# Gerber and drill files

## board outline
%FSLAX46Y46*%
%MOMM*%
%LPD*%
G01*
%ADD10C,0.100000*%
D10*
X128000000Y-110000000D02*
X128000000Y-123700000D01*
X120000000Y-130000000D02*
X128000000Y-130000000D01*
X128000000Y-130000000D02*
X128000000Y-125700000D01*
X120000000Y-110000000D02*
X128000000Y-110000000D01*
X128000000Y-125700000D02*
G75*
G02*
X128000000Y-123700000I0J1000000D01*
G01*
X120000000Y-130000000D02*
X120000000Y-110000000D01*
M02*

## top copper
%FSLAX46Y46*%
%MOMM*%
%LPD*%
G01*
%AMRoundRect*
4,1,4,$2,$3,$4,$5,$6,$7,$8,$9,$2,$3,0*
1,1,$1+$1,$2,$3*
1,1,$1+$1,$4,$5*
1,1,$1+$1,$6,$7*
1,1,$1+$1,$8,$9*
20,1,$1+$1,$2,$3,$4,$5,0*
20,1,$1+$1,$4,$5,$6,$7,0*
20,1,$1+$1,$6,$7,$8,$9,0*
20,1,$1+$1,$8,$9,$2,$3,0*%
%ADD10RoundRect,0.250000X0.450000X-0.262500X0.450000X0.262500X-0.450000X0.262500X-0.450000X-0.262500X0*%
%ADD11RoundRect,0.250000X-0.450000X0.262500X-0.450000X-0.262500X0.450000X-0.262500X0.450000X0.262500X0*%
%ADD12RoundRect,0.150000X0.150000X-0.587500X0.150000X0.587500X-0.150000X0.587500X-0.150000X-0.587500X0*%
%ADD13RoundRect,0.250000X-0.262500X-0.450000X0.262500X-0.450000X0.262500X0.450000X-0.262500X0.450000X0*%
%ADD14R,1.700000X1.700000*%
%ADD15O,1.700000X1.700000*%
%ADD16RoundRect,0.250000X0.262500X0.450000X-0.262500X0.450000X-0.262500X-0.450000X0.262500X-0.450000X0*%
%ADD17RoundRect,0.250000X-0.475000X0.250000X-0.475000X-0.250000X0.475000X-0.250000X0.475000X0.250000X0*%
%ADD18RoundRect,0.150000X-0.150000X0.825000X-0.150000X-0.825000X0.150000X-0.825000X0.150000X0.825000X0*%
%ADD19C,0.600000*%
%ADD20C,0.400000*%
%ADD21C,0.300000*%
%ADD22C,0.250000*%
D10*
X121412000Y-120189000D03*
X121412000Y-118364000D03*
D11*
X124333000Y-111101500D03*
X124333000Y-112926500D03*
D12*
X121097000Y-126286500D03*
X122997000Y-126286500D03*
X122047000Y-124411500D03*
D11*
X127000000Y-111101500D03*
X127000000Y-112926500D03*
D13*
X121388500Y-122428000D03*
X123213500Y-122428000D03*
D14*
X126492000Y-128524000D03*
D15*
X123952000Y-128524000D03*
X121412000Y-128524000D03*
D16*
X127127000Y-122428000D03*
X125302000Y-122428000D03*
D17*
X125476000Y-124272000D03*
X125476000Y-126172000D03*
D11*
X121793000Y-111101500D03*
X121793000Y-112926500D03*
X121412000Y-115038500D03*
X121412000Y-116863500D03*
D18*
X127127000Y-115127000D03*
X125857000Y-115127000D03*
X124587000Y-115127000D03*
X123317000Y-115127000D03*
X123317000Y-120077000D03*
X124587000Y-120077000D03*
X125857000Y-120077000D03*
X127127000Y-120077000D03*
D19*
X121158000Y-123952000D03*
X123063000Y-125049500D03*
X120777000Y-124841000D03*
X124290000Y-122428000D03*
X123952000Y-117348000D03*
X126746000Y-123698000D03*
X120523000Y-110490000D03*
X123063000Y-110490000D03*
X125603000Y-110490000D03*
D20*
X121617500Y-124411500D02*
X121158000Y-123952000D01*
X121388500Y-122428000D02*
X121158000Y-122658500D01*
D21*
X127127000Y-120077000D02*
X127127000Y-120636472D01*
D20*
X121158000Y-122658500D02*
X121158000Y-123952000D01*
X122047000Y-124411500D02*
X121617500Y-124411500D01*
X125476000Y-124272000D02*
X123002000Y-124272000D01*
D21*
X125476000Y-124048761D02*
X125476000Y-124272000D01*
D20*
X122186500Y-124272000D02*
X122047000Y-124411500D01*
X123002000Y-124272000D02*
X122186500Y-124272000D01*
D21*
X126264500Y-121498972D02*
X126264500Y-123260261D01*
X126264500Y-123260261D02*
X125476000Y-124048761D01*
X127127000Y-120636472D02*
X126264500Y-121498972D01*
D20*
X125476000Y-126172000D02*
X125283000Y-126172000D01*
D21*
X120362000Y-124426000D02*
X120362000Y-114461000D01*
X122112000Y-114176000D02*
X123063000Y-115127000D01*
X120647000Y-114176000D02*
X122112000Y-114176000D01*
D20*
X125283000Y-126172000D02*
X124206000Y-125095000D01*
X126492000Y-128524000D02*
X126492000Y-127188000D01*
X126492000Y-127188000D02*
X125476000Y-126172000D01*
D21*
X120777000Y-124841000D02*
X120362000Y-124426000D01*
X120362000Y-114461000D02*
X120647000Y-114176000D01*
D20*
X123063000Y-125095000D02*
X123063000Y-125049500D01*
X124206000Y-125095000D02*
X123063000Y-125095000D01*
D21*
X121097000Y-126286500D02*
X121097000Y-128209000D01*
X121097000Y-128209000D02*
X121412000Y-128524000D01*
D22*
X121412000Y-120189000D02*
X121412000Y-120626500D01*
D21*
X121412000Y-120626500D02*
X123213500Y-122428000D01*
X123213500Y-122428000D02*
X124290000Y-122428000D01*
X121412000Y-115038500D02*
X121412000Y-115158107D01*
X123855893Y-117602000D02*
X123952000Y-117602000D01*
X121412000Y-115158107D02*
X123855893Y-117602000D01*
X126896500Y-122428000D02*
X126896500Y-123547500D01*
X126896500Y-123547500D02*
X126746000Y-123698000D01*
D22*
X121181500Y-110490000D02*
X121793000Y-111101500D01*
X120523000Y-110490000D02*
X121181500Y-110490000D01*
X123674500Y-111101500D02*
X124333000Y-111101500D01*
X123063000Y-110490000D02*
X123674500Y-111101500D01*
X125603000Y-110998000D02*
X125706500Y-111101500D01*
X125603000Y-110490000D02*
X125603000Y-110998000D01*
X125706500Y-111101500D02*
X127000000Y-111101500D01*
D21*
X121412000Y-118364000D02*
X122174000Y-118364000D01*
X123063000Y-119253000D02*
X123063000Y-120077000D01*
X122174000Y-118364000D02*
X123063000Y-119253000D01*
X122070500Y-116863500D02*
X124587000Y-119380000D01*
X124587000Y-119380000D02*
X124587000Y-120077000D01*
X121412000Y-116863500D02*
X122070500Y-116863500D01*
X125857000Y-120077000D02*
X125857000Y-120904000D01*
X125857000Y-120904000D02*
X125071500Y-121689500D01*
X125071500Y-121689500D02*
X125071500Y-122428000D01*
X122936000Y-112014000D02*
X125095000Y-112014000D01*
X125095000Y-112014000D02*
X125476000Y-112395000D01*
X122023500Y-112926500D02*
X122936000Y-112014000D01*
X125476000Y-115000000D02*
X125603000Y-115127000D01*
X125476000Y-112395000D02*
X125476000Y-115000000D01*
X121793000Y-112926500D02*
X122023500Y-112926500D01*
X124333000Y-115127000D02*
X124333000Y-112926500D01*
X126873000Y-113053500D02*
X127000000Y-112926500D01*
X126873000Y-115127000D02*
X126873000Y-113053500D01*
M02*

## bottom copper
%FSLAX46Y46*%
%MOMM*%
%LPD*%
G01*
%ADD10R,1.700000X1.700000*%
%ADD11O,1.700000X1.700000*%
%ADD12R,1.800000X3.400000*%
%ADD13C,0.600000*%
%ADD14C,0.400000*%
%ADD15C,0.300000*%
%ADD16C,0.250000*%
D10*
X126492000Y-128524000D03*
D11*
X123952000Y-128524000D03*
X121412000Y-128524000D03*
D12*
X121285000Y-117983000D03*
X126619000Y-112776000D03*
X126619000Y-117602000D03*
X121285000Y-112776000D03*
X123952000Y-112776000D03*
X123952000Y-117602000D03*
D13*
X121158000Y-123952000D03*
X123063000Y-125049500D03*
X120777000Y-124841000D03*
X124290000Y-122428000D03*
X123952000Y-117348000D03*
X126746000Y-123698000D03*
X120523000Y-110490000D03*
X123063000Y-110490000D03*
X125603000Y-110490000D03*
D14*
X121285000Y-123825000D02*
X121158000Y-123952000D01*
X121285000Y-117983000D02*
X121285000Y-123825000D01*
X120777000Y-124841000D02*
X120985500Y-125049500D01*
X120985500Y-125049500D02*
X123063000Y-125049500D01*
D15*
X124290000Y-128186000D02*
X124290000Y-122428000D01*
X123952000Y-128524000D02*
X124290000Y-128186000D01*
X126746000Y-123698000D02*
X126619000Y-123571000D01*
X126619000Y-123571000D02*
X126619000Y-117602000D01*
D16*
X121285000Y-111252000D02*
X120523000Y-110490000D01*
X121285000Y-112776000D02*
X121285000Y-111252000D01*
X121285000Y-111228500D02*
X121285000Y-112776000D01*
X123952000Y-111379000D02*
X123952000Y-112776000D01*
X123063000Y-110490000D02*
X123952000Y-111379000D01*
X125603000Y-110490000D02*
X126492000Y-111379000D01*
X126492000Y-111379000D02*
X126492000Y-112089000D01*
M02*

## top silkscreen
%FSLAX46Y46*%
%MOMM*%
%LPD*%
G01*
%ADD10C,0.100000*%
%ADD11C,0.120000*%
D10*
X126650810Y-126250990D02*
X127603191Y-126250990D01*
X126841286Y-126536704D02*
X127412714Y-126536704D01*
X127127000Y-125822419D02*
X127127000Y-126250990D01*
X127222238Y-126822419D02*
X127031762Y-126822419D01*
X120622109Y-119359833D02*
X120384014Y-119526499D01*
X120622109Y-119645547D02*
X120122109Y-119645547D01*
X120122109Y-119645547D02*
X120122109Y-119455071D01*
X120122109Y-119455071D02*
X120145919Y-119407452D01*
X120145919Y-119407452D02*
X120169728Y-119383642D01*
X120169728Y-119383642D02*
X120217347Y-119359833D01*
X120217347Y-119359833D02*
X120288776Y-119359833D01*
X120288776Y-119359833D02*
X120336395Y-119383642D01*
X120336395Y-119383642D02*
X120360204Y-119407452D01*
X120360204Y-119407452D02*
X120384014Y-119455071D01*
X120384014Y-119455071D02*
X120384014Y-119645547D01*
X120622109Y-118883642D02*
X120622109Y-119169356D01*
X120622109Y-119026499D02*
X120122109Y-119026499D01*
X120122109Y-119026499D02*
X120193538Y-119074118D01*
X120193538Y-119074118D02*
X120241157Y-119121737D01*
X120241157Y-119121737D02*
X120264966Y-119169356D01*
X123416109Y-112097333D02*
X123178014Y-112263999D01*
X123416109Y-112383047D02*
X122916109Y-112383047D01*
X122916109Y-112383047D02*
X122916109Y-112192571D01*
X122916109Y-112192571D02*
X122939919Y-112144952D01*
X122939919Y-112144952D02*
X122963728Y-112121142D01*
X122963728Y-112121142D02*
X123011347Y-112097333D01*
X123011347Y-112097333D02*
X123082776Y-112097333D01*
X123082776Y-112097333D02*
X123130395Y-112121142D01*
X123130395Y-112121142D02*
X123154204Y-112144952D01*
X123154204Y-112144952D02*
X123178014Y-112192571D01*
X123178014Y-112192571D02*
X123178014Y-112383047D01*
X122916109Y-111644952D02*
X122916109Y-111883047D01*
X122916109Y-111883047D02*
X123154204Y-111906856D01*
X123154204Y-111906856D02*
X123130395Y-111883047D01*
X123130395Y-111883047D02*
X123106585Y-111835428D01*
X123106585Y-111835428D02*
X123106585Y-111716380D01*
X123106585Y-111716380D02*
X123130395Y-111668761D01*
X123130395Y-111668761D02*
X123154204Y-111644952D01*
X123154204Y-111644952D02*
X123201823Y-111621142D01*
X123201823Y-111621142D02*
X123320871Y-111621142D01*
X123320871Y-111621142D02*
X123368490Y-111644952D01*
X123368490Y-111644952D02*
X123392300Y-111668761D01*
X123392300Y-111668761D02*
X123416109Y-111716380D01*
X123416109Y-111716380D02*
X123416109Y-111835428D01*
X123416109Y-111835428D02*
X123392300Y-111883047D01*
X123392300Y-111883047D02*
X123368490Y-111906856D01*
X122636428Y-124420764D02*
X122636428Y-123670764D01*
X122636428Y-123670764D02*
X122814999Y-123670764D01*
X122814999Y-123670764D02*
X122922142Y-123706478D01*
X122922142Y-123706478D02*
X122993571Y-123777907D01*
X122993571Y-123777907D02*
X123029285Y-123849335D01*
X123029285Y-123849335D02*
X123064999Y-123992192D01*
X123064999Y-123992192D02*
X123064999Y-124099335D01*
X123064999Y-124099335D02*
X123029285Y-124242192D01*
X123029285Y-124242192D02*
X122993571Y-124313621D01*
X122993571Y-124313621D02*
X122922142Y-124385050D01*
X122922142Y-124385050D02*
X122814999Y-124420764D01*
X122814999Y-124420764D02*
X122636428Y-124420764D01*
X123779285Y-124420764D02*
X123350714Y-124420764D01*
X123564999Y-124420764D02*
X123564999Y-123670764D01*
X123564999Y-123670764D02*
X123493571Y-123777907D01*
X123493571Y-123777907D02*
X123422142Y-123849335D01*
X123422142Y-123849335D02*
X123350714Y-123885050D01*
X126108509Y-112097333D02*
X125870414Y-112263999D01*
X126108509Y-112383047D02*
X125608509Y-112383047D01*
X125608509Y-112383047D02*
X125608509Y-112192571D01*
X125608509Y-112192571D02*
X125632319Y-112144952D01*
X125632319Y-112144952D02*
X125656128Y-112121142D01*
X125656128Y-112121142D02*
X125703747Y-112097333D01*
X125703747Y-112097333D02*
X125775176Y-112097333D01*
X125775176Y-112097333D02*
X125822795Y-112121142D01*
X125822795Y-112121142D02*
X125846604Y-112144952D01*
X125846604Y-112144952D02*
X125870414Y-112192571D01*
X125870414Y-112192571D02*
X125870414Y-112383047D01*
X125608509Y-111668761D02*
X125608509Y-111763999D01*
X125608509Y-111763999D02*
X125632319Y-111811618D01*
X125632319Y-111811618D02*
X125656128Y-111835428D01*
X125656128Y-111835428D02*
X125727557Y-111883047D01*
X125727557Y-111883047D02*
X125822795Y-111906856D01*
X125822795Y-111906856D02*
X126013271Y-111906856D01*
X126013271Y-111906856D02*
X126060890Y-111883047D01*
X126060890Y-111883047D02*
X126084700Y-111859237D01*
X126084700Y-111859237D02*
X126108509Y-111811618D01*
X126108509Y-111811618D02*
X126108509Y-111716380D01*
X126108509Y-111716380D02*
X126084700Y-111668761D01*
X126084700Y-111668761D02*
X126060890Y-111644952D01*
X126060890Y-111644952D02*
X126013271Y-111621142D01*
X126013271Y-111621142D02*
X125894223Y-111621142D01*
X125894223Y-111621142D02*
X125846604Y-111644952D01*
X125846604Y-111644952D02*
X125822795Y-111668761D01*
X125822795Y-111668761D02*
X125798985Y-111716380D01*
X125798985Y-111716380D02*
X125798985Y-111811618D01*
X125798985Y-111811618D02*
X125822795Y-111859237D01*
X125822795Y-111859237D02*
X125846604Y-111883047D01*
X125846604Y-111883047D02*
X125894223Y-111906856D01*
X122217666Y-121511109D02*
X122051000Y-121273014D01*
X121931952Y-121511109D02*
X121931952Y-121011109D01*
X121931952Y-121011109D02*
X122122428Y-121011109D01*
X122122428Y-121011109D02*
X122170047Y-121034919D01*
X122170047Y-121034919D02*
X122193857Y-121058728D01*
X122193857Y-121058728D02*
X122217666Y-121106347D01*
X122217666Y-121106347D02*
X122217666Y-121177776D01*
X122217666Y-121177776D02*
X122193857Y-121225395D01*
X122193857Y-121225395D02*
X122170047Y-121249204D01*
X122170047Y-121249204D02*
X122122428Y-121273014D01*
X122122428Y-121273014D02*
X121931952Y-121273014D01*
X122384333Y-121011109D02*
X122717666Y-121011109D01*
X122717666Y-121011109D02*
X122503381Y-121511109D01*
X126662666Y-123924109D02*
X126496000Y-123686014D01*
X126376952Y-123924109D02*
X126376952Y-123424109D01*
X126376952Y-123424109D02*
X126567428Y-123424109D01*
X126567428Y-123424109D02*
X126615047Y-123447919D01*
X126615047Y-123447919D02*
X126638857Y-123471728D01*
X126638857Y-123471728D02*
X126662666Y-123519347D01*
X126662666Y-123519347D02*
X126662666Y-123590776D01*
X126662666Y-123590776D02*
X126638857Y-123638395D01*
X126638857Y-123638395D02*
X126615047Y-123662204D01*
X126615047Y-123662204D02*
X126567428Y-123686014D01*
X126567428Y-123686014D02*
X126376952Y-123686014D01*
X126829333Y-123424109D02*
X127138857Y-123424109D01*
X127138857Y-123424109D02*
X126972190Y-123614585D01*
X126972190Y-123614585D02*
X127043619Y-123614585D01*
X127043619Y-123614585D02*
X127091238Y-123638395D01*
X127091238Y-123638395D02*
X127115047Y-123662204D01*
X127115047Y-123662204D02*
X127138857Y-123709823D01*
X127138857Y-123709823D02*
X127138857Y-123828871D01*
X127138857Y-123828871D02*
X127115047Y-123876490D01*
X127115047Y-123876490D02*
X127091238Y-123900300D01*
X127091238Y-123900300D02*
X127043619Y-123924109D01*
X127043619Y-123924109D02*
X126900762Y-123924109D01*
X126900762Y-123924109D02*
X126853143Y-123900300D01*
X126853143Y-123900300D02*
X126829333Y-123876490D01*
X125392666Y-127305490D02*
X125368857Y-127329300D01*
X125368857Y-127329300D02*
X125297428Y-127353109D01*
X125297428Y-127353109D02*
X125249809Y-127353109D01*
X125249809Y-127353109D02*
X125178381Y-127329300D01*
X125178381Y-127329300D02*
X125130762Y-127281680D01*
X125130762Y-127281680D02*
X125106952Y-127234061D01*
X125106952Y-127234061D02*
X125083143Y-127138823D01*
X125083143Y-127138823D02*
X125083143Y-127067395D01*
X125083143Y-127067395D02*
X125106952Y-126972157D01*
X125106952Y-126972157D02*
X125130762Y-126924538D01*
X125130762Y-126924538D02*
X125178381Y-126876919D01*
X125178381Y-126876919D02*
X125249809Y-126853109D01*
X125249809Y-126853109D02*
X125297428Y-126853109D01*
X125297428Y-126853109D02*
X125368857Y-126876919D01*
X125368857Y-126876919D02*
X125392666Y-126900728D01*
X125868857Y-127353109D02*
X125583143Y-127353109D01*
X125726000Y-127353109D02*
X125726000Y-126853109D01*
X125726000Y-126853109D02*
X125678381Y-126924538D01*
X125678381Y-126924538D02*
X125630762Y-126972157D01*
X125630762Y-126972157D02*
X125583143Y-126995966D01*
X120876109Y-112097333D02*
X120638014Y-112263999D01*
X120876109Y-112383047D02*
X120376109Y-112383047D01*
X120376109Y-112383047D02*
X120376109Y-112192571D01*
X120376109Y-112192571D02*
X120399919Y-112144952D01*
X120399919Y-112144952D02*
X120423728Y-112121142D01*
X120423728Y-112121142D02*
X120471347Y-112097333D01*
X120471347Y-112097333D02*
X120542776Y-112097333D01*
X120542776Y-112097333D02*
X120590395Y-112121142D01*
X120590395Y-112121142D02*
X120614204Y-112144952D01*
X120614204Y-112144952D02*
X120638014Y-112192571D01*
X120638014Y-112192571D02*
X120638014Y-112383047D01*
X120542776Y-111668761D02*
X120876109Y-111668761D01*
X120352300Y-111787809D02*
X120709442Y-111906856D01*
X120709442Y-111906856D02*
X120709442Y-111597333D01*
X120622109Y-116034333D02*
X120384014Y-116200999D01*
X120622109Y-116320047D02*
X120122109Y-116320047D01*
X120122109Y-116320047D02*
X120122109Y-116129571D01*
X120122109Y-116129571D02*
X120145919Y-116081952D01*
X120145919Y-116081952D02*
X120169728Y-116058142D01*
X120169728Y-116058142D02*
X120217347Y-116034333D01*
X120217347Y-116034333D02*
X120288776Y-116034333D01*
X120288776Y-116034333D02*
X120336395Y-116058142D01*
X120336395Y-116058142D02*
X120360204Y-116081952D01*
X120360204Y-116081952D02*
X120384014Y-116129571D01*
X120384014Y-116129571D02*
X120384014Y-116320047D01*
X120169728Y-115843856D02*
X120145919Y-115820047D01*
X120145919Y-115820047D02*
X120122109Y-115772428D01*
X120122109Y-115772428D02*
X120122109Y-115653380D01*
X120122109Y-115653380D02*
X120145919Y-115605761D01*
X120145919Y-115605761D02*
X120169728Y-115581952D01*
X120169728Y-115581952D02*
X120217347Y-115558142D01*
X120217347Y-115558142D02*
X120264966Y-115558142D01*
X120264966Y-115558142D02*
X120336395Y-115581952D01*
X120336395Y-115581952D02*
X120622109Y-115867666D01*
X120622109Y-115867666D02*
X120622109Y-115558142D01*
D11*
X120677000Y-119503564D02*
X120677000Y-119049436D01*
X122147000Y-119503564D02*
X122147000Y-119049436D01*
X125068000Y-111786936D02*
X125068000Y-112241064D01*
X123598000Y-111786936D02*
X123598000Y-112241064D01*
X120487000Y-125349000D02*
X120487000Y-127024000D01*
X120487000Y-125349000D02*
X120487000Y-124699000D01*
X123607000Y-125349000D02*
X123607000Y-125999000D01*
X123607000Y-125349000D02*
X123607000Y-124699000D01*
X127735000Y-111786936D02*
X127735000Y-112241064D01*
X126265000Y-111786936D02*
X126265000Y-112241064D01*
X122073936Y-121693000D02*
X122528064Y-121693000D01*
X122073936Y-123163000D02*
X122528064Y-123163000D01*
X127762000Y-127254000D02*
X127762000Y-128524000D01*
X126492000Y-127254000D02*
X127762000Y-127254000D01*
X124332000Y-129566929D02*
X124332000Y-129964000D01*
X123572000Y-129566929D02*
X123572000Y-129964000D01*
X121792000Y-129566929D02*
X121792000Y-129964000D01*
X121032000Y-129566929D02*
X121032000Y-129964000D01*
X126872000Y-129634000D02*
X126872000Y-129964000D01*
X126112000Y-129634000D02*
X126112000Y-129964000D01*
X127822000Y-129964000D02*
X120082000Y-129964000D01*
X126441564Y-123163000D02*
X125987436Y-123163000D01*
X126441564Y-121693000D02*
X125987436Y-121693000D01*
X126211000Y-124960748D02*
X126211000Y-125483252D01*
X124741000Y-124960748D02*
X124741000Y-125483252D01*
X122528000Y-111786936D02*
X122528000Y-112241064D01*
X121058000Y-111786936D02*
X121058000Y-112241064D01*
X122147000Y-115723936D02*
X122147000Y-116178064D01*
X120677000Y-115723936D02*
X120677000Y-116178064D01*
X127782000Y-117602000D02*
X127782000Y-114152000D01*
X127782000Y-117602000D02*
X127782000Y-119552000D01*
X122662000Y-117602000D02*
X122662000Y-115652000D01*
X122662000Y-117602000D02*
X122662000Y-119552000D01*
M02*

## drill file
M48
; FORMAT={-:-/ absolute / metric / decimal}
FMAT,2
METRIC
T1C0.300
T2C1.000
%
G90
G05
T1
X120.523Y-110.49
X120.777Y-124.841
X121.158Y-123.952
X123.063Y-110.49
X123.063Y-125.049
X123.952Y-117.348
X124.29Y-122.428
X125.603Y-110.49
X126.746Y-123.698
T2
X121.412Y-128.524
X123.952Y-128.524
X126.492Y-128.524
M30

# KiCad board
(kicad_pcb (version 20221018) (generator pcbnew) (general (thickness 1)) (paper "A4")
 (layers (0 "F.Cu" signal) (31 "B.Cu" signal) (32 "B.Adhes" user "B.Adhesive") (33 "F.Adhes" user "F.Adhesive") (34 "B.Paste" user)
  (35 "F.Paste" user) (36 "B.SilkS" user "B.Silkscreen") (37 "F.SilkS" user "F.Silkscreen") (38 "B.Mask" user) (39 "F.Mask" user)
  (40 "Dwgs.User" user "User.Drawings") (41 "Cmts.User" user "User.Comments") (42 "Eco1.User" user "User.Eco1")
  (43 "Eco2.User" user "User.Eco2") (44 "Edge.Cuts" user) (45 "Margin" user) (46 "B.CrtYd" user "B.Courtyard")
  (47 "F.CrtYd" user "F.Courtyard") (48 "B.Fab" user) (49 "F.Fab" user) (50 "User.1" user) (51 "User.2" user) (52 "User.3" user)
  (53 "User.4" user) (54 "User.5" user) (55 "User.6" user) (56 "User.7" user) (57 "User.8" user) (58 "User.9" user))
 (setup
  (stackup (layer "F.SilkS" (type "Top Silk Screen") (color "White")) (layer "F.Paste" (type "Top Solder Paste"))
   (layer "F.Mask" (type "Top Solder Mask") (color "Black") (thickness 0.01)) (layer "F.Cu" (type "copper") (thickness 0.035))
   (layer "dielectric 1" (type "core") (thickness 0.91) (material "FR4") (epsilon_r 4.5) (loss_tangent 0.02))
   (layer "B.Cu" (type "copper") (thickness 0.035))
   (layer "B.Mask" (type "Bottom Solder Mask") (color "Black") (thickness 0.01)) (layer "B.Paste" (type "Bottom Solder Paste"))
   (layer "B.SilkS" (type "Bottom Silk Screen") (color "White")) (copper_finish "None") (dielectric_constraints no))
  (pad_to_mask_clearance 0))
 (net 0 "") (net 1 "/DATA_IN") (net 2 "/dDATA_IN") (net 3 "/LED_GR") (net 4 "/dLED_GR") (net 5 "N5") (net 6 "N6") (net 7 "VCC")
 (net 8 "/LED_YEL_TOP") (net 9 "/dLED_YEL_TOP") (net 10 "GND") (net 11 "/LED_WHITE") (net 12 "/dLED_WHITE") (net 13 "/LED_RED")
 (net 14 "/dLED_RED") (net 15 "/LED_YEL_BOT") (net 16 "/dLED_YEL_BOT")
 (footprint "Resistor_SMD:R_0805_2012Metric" (layer "F.Cu") (at 121.412 119.2765 90)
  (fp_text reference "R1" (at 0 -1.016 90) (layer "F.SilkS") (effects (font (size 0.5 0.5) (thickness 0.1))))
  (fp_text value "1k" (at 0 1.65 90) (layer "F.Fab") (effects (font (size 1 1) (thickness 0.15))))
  (fp_line (start -0.227064 -0.735) (end 0.227064 -0.735) (stroke (width 0.12) (type solid)) (layer "F.SilkS"))
  (fp_line (start -0.227064 0.735) (end 0.227064 0.735) (stroke (width 0.12) (type solid)) (layer "F.SilkS"))
  (pad "1" smd roundrect (at -0.9125 0 90) (size 1.025 1.4) (layers "F.Cu" "F.Paste" "F.Mask") (roundrect_rratio 0.243902)
   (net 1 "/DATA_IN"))
  (pad "2" smd roundrect (at 0.9125 0 90) (size 1.025 1.4) (layers "F.Cu" "F.Paste" "F.Mask") (roundrect_rratio 0.243902)
   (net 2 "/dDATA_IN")))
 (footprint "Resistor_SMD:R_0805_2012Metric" (layer "F.Cu") (at 124.333 112.014 -90)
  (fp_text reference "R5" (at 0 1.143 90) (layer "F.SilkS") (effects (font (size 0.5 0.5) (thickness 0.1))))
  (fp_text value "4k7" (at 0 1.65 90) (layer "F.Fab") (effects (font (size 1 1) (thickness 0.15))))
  (fp_line (start -0.227064 -0.735) (end 0.227064 -0.735) (stroke (width 0.12) (type solid)) (layer "F.SilkS"))
  (fp_line (start -0.227064 0.735) (end 0.227064 0.735) (stroke (width 0.12) (type solid)) (layer "F.SilkS"))
  (pad "1" smd roundrect (at -0.9125 0 270) (size 1.025 1.4) (layers "F.Cu" "F.Paste" "F.Mask") (roundrect_rratio 0.243902)
   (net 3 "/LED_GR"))
  (pad "2" smd roundrect (at 0.9125 0 270) (size 1.025 1.4) (layers "F.Cu" "F.Paste" "F.Mask") (roundrect_rratio 0.243902)
   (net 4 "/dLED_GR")))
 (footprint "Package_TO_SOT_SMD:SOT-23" (layer "F.Cu") (at 122.047 125.349 90)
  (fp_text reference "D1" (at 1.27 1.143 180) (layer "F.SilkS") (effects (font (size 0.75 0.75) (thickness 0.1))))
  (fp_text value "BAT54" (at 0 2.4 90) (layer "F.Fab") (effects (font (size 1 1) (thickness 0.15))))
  (fp_line (start 0 -1.56) (end -1.675 -1.56) (stroke (width 0.12) (type solid)) (layer "F.SilkS"))
  (fp_line (start 0 -1.56) (end 0.65 -1.56) (stroke (width 0.12) (type solid)) (layer "F.SilkS"))
  (fp_line (start 0 1.56) (end -0.65 1.56) (stroke (width 0.12) (type solid)) (layer "F.SilkS"))
  (fp_line (start 0 1.56) (end 0.65 1.56) (stroke (width 0.12) (type solid)) (layer "F.SilkS"))
  (pad "1" smd roundrect (at -0.9375 -0.95 90) (size 1.475 0.6) (layers "F.Cu" "F.Paste" "F.Mask") (roundrect_rratio 0.25) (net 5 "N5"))
  (pad "2" smd roundrect (at -0.9375 0.95 90) (size 1.475 0.6) (layers "F.Cu" "F.Paste" "F.Mask") (roundrect_rratio 0.25) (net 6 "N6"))
  (pad "3" smd roundrect (at 0.9375 0 90) (size 1.475 0.6) (layers "F.Cu" "F.Paste" "F.Mask") (roundrect_rratio 0.25) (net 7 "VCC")))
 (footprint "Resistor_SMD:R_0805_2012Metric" (layer "F.Cu") (at 127 112.014 -90)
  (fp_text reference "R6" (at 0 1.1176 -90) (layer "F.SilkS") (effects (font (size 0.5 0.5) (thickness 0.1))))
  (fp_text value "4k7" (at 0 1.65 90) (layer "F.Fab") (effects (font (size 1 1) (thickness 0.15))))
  (fp_line (start -0.227064 -0.735) (end 0.227064 -0.735) (stroke (width 0.12) (type solid)) (layer "F.SilkS"))
  (fp_line (start -0.227064 0.735) (end 0.227064 0.735) (stroke (width 0.12) (type solid)) (layer "F.SilkS"))
  (pad "1" smd roundrect (at -0.9125 0 270) (size 1.025 1.4) (layers "F.Cu" "F.Paste" "F.Mask") (roundrect_rratio 0.243902)
   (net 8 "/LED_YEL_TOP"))
  (pad "2" smd roundrect (at 0.9125 0 270) (size 1.025 1.4) (layers "F.Cu" "F.Paste" "F.Mask") (roundrect_rratio 0.243902)
   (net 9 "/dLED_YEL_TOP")))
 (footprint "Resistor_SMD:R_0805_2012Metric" (layer "F.Cu") (at 122.301 122.428)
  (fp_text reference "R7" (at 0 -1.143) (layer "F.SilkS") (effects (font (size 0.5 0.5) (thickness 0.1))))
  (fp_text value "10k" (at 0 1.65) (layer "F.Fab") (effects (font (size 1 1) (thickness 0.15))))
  (fp_line (start -0.227064 -0.735) (end 0.227064 -0.735) (stroke (width 0.12) (type solid)) (layer "F.SilkS"))
  (fp_line (start -0.227064 0.735) (end 0.227064 0.735) (stroke (width 0.12) (type solid)) (layer "F.SilkS"))
  (pad "1" smd roundrect (at -0.9125 0) (size 1.025 1.4) (layers "F.Cu" "F.Paste" "F.Mask") (roundrect_rratio 0.243902) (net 7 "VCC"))
  (pad "2" smd roundrect (at 0.9125 0) (size 1.025 1.4) (layers "F.Cu" "F.Paste" "F.Mask") (roundrect_rratio 0.243902) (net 1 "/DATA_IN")))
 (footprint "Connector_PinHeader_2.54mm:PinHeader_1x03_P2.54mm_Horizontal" (layer "F.Cu") (at 126.492 128.524 -90)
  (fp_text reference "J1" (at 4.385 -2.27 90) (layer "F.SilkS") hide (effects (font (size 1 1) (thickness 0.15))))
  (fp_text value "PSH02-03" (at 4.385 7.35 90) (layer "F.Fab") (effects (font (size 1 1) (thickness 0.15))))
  (fp_line (start -1.27 -1.27) (end 0 -1.27) (stroke (width 0.12) (type solid)) (layer "F.SilkS"))
  (fp_line (start -1.27 0) (end -1.27 -1.27) (stroke (width 0.12) (type solid)) (layer "F.SilkS"))
  (fp_line (start 1.042929 2.16) (end 1.44 2.16) (stroke (width 0.12) (type solid)) (layer "F.SilkS"))
  (fp_line (start 1.042929 2.92) (end 1.44 2.92) (stroke (width 0.12) (type solid)) (layer "F.SilkS"))
  (fp_line (start 1.042929 4.7) (end 1.44 4.7) (stroke (width 0.12) (type solid)) (layer "F.SilkS"))
  (fp_line (start 1.042929 5.46) (end 1.44 5.46) (stroke (width 0.12) (type solid)) (layer "F.SilkS"))
  (fp_line (start 1.11 -0.38) (end 1.44 -0.38) (stroke (width 0.12) (type solid)) (layer "F.SilkS"))
  (fp_line (start 1.11 0.38) (end 1.44 0.38) (stroke (width 0.12) (type solid)) (layer "F.SilkS"))
  (fp_line (start 1.44 -1.33) (end 1.44 6.41) (stroke (width 0.12) (type solid)) (layer "F.SilkS"))
  (pad "1" thru_hole rect (at 0 0 270) (size 1.7 1.7) (drill 1) (layers "*.Cu" "*.Mask") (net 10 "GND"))
  (pad "2" thru_hole oval (at 0 2.54 270) (size 1.7 1.7) (drill 1) (layers "*.Cu" "*.Mask") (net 1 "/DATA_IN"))
  (pad "3" thru_hole oval (at 0 5.08 270) (size 1.7 1.7) (drill 1) (layers "*.Cu" "*.Mask") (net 5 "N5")))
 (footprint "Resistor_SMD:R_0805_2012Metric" (layer "F.Cu") (at 126.2145 122.428 180)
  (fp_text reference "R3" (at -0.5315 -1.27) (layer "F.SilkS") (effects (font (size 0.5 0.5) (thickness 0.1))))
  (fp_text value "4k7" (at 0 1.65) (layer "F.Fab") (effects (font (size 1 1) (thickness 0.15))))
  (fp_line (start -0.227064 -0.735) (end 0.227064 -0.735) (stroke (width 0.12) (type solid)) (layer "F.SilkS"))
  (fp_line (start -0.227064 0.735) (end 0.227064 0.735) (stroke (width 0.12) (type solid)) (layer "F.SilkS"))
  (pad "1" smd roundrect (at -0.9125 0 180) (size 1.025 1.4) (layers "F.Cu" "F.Paste" "F.Mask") (roundrect_rratio 0.243902)
   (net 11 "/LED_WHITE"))
  (pad "2" smd roundrect (at 0.9125 0 180) (size 1.025 1.4) (layers "F.Cu" "F.Paste" "F.Mask") (roundrect_rratio 0.243902)
   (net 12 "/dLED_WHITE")))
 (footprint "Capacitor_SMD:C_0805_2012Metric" (layer "F.Cu") (at 125.476 125.222 -90)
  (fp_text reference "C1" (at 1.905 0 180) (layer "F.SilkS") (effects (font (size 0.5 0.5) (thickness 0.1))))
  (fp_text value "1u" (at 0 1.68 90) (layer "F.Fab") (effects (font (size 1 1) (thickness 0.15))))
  (fp_line (start -0.261252 -0.735) (end 0.261252 -0.735) (stroke (width 0.12) (type solid)) (layer "F.SilkS"))
  (fp_line (start -0.261252 0.735) (end 0.261252 0.735) (stroke (width 0.12) (type solid)) (layer "F.SilkS"))
  (pad "1" smd roundrect (at -0.95 0 270) (size 1 1.45) (layers "F.Cu" "F.Paste" "F.Mask") (roundrect_rratio 0.25) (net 7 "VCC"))
  (pad "2" smd roundrect (at 0.95 0 270) (size 1 1.45) (layers "F.Cu" "F.Paste" "F.Mask") (roundrect_rratio 0.25) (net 10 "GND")))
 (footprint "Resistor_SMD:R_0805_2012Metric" (layer "F.Cu") (at 121.793 112.014 -90)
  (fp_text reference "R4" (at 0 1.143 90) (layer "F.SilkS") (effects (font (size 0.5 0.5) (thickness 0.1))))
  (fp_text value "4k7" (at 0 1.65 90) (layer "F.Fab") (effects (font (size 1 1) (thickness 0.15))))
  (fp_line (start -0.227064 -0.735) (end 0.227064 -0.735) (stroke (width 0.12) (type solid)) (layer "F.SilkS"))
  (fp_line (start -0.227064 0.735) (end 0.227064 0.735) (stroke (width 0.12) (type solid)) (layer "F.SilkS"))
  (pad "1" smd roundrect (at -0.9125 0 270) (size 1.025 1.4) (layers "F.Cu" "F.Paste" "F.Mask") (roundrect_rratio 0.243902)
   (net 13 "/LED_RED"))
  (pad "2" smd roundrect (at 0.9125 0 270) (size 1.025 1.4) (layers "F.Cu" "F.Paste" "F.Mask") (roundrect_rratio 0.243902)
   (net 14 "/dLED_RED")))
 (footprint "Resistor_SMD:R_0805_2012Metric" (layer "F.Cu") (at 121.412 115.951 -90)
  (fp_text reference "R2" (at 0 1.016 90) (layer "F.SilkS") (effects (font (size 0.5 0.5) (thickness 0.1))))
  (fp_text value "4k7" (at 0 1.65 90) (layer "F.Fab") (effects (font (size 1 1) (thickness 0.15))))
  (fp_line (start -0.227064 -0.735) (end 0.227064 -0.735) (stroke (width 0.12) (type solid)) (layer "F.SilkS"))
  (fp_line (start -0.227064 0.735) (end 0.227064 0.735) (stroke (width 0.12) (type solid)) (layer "F.SilkS"))
  (pad "1" smd roundrect (at -0.9125 0 270) (size 1.025 1.4) (layers "F.Cu" "F.Paste" "F.Mask") (roundrect_rratio 0.243902)
   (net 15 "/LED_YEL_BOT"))
  (pad "2" smd roundrect (at 0.9125 0 270) (size 1.025 1.4) (layers "F.Cu" "F.Paste" "F.Mask") (roundrect_rratio 0.243902)
   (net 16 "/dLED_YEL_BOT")))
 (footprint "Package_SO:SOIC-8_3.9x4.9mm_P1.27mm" (layer "F.Cu") (at 125.222 117.602 -90)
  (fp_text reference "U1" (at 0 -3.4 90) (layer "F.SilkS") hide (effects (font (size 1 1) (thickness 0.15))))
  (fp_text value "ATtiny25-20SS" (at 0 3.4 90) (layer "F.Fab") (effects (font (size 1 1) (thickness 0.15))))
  (fp_line (start 0 -2.56) (end -3.45 -2.56) (stroke (width 0.12) (type solid)) (layer "F.SilkS"))
  (fp_line (start 0 -2.56) (end 1.95 -2.56) (stroke (width 0.12) (type solid)) (layer "F.SilkS"))
  (fp_line (start 0 2.56) (end -1.95 2.56) (stroke (width 0.12) (type solid)) (layer "F.SilkS"))
  (fp_line (start 0 2.56) (end 1.95 2.56) (stroke (width 0.12) (type solid)) (layer "F.SilkS"))
  (pad "1" smd roundrect (at -2.475 -1.905 270) (size 1.95 0.6) (layers "F.Cu" "F.Paste" "F.Mask") (roundrect_rratio 0.25)
   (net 9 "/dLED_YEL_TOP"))
  (pad "2" smd roundrect (at -2.475 -0.635 270) (size 1.95 0.6) (layers "F.Cu" "F.Paste" "F.Mask") (roundrect_rratio 0.25)
   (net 14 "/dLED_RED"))
  (pad "3" smd roundrect (at -2.475 0.635 270) (size 1.95 0.6) (layers "F.Cu" "F.Paste" "F.Mask") (roundrect_rratio 0.25) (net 4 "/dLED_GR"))
  (pad "4" smd roundrect (at -2.475 1.905 270) (size 1.95 0.6) (layers "F.Cu" "F.Paste" "F.Mask") (roundrect_rratio 0.25) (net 10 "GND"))
  (pad "5" smd roundrect (at 2.475 1.905 270) (size 1.95 0.6) (layers "F.Cu" "F.Paste" "F.Mask") (roundrect_rratio 0.25) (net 2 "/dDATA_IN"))
  (pad "6" smd roundrect (at 2.475 0.635 270) (size 1.95 0.6) (layers "F.Cu" "F.Paste" "F.Mask") (roundrect_rratio 0.25)
   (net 16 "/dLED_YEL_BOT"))
  (pad "7" smd roundrect (at 2.475 -0.635 270) (size 1.95 0.6) (layers "F.Cu" "F.Paste" "F.Mask") (roundrect_rratio 0.25)
   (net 12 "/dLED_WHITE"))
  (pad "8" smd roundrect (at 2.475 -1.905 270) (size 1.95 0.6) (layers "F.Cu" "F.Paste" "F.Mask") (roundrect_rratio 0.25) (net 7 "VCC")))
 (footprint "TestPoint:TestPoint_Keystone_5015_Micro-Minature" (layer "B.Cu") (at 121.285 117.983 -90)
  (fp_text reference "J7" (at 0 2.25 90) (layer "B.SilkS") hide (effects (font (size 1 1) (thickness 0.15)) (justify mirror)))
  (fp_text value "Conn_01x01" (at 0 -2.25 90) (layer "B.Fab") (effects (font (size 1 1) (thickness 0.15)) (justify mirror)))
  (pad "1" smd rect (at 0 0 270) (size 3.4 1.8) (layers "B.Cu" "B.Paste" "B.Mask") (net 7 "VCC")))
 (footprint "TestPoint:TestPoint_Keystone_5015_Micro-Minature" (layer "B.Cu") (at 126.619 112.776 -90)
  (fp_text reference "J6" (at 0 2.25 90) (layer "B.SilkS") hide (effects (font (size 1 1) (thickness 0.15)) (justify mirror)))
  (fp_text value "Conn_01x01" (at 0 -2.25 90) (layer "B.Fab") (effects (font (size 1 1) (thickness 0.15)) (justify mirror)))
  (pad "1" smd rect (at 0 0 270) (size 3.4 1.8) (layers "B.Cu" "B.Paste" "B.Mask") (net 8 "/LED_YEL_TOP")))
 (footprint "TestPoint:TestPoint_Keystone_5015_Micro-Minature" (layer "B.Cu") (at 126.619 117.602 -90)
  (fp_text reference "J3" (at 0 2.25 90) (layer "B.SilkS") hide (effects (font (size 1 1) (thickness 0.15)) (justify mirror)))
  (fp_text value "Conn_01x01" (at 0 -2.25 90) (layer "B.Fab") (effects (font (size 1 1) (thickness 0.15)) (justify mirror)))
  (pad "1" smd rect (at 0 0 270) (size 3.4 1.8) (layers "B.Cu" "B.Paste" "B.Mask") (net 11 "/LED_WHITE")))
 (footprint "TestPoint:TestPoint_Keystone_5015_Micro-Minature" (layer "B.Cu") (at 121.285 112.776 -90)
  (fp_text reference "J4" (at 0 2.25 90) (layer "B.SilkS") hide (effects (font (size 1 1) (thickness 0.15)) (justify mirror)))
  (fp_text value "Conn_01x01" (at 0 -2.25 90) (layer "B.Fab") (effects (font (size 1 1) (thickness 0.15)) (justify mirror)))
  (pad "1" smd rect (at 0 0 270) (size 3.4 1.8) (layers "B.Cu" "B.Paste" "B.Mask") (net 13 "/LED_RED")))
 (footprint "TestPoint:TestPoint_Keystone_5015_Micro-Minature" (layer "B.Cu") (at 123.952 112.776 -90)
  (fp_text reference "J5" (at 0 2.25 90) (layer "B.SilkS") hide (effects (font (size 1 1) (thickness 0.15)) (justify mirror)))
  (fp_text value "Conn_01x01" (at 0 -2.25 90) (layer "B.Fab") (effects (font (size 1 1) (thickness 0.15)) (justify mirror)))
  (pad "1" smd rect (at 0 0 270) (size 3.4 1.8) (layers "B.Cu" "B.Paste" "B.Mask") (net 3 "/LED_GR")))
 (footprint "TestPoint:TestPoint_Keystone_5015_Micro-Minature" (layer "B.Cu") (at 123.952 117.602 -90)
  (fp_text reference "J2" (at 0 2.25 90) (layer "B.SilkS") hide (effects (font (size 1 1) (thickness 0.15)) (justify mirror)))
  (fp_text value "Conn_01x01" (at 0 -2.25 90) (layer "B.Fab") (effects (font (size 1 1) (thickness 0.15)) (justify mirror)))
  (pad "1" smd rect (at 0 0 270) (size 3.4 1.8) (layers "B.Cu" "B.Paste" "B.Mask") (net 15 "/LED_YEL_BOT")))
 (gr_line (start 128 110) (end 128 123.7) (stroke (width 0.1) (type solid)) (layer "Edge.Cuts"))
 (gr_line (start 120 130) (end 128 130) (stroke (width 0.1) (type solid)) (layer "Edge.Cuts"))
 (gr_line (start 128 130) (end 128 125.7) (stroke (width 0.1) (type solid)) (layer "Edge.Cuts"))
 (gr_line (start 120 110) (end 128 110) (stroke (width 0.1) (type solid)) (layer "Edge.Cuts"))
 (gr_arc (start 128 125.7) (mid 127 124.7) (end 128 123.7) (stroke (width 0.1) (type solid)) (layer "Edge.Cuts"))
 (gr_line (start 120 130) (end 120 110) (stroke (width 0.1) (type solid)) (layer "Edge.Cuts"))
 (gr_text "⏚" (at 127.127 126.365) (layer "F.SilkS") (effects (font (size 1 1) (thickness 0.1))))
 (segment (start 121.6175 124.4115) (end 121.158 123.952) (width 0.4) (layer "F.Cu") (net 7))
 (segment (start 121.3885 122.428) (end 121.158 122.6585) (width 0.4) (layer "F.Cu") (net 7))
 (segment (start 127.127 120.077) (end 127.127 120.636472) (width 0.3) (layer "F.Cu") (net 7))
 (segment (start 121.158 122.6585) (end 121.158 123.952) (width 0.4) (layer "F.Cu") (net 7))
 (segment (start 122.047 124.4115) (end 121.6175 124.4115) (width 0.4) (layer "F.Cu") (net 7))
 (segment (start 125.476 124.272) (end 123.002 124.272) (width 0.4) (layer "F.Cu") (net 7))
 (segment (start 125.476 124.048761) (end 125.476 124.272) (width 0.3) (layer "F.Cu") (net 7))
 (segment (start 122.1865 124.272) (end 122.047 124.4115) (width 0.4) (layer "F.Cu") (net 7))
 (segment (start 123.002 124.272) (end 122.1865 124.272) (width 0.4) (layer "F.Cu") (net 7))
 (segment (start 126.2645 121.498972) (end 126.2645 123.260261) (width 0.3) (layer "F.Cu") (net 7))
 (segment (start 126.2645 123.260261) (end 125.476 124.048761) (width 0.3) (layer "F.Cu") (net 7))
 (segment (start 127.127 120.636472) (end 126.2645 121.498972) (width 0.3) (layer "F.Cu") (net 7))
 (via (at 121.158 123.952) (size 0.6) (drill 0.3) (layers "F.Cu" "B.Cu") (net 7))
 (segment (start 121.285 123.825) (end 121.158 123.952) (width 0.4) (layer "B.Cu") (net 7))
 (segment (start 121.285 117.983) (end 121.285 123.825) (width 0.4) (layer "B.Cu") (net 7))
 (segment (start 125.476 126.172) (end 125.283 126.172) (width 0.4) (layer "F.Cu") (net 10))
 (segment (start 120.362 124.426) (end 120.362 114.461) (width 0.3) (layer "F.Cu") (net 10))
 (segment (start 122.112 114.176) (end 123.063 115.127) (width 0.3) (layer "F.Cu") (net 10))
 (segment (start 120.647 114.176) (end 122.112 114.176) (width 0.3) (layer "F.Cu") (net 10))
 (segment (start 125.283 126.172) (end 124.206 125.095) (width 0.4) (layer "F.Cu") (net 10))
 (segment (start 126.492 128.524) (end 126.492 127.188) (width 0.4) (layer "F.Cu") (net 10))
 (segment (start 126.492 127.188) (end 125.476 126.172) (width 0.4) (layer "F.Cu") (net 10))
 (segment (start 120.777 124.841) (end 120.362 124.426) (width 0.3) (layer "F.Cu") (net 10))
 (segment (start 120.362 114.461) (end 120.647 114.176) (width 0.3) (layer "F.Cu") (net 10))
 (segment (start 123.063 125.095) (end 123.063 125.0495) (width 0.4) (layer "F.Cu") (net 10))
 (segment (start 124.206 125.095) (end 123.063 125.095) (width 0.4) (layer "F.Cu") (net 10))
 (via (at 123.063 125.0495) (size 0.6) (drill 0.3) (layers "F.Cu" "B.Cu") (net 10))
 (via (at 120.777 124.841) (size 0.6) (drill 0.3) (layers "F.Cu" "B.Cu") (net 10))
 (segment (start 120.777 124.841) (end 120.9855 125.0495) (width 0.4) (layer "B.Cu") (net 10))
 (segment (start 120.9855 125.0495) (end 123.063 125.0495) (width 0.4) (layer "B.Cu") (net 10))
 (segment (start 121.097 126.2865) (end 121.097 128.209) (width 0.3) (layer "F.Cu") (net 5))
 (segment (start 121.097 128.209) (end 121.412 128.524) (width 0.3) (layer "F.Cu") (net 5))
 (segment (start 121.412 120.189) (end 121.412 120.6265) (width 0.25) (layer "F.Cu") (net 1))
 (segment (start 121.412 120.6265) (end 123.2135 122.428) (width 0.3) (layer "F.Cu") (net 1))
 (segment (start 123.2135 122.428) (end 124.29 122.428) (width 0.3) (layer "F.Cu") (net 1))
 (via (at 124.29 122.428) (size 0.6) (drill 0.3) (layers "F.Cu" "B.Cu") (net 1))
 (segment (start 124.29 128.186) (end 124.29 122.428) (width 0.3) (layer "B.Cu") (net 1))
 (segment (start 123.952 128.524) (end 124.29 128.186) (width 0.3) (layer "B.Cu") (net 1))
 (segment (start 121.412 115.0385) (end 121.412 115.158107) (width 0.3) (layer "F.Cu") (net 15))
 (segment (start 123.855893 117.602) (end 123.952 117.602) (width 0.3) (layer "F.Cu") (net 15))
 (segment (start 121.412 115.158107) (end 123.855893 117.602) (width 0.3) (layer "F.Cu") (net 15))
 (via (at 123.952 117.348) (size 0.6) (drill 0.3) (layers "F.Cu" "B.Cu") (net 15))
 (segment (start 126.8965 122.428) (end 126.8965 123.5475) (width 0.3) (layer "F.Cu") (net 11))
 (segment (start 126.8965 123.5475) (end 126.746 123.698) (width 0.3) (layer "F.Cu") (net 11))
 (via (at 126.746 123.698) (size 0.6) (drill 0.3) (layers "F.Cu" "B.Cu") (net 11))
 (segment (start 126.746 123.698) (end 126.619 123.571) (width 0.3) (layer "B.Cu") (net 11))
 (segment (start 126.619 123.571) (end 126.619 117.602) (width 0.3) (layer "B.Cu") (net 11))
 (segment (start 121.1815 110.49) (end 121.793 111.1015) (width 0.25) (layer "F.Cu") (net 13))
 (segment (start 120.523 110.49) (end 121.1815 110.49) (width 0.25) (layer "F.Cu") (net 13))
 (via (at 120.523 110.49) (size 0.6) (drill 0.3) (layers "F.Cu" "B.Cu") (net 13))
 (segment (start 121.285 111.252) (end 120.523 110.49) (width 0.25) (layer "B.Cu") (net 13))
 (segment (start 121.285 112.776) (end 121.285 111.252) (width 0.25) (layer "B.Cu") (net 13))
 (segment (start 121.285 111.2285) (end 121.285 112.776) (width 0.25) (layer "B.Cu") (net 13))
 (segment (start 123.6745 111.1015) (end 124.333 111.1015) (width 0.25) (layer "F.Cu") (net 3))
 (segment (start 123.063 110.49) (end 123.6745 111.1015) (width 0.25) (layer "F.Cu") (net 3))
 (via (at 123.063 110.49) (size 0.6) (drill 0.3) (layers "F.Cu" "B.Cu") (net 3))
 (segment (start 123.952 111.379) (end 123.952 112.776) (width 0.25) (layer "B.Cu") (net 3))
 (segment (start 123.063 110.49) (end 123.952 111.379) (width 0.25) (layer "B.Cu") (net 3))
 (segment (start 125.603 110.998) (end 125.7065 111.1015) (width 0.25) (layer "F.Cu") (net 8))
 (segment (start 125.603 110.49) (end 125.603 110.998) (width 0.25) (layer "F.Cu") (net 8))
 (segment (start 125.7065 111.1015) (end 127 111.1015) (width 0.25) (layer "F.Cu") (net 8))
 (via (at 125.603 110.49) (size 0.6) (drill 0.3) (layers "F.Cu" "B.Cu") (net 8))
 (segment (start 125.603 110.49) (end 126.492 111.379) (width 0.25) (layer "B.Cu") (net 8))
 (segment (start 126.492 111.379) (end 126.492 112.089) (width 0.25) (layer "B.Cu") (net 8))
 (segment (start 121.412 118.364) (end 122.174 118.364) (width 0.3) (layer "F.Cu") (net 2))
 (segment (start 123.063 119.253) (end 123.063 120.077) (width 0.3) (layer "F.Cu") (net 2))
 (segment (start 122.174 118.364) (end 123.063 119.253) (width 0.3) (layer "F.Cu") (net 2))
 (segment (start 122.0705 116.8635) (end 124.587 119.38) (width 0.3) (layer "F.Cu") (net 16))
 (segment (start 124.587 119.38) (end 124.587 120.077) (width 0.3) (layer "F.Cu") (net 16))
 (segment (start 121.412 116.8635) (end 122.0705 116.8635) (width 0.3) (layer "F.Cu") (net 16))
 (segment (start 125.857 120.077) (end 125.857 120.904) (width 0.3) (layer "F.Cu") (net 12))
 (segment (start 125.857 120.904) (end 125.0715 121.6895) (width 0.3) (layer "F.Cu") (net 12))
 (segment (start 125.0715 121.6895) (end 125.0715 122.428) (width 0.3) (layer "F.Cu") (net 12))
 (segment (start 122.936 112.014) (end 125.095 112.014) (width 0.3) (layer "F.Cu") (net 14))
 (segment (start 125.095 112.014) (end 125.476 112.395) (width 0.3) (layer "F.Cu") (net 14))
 (segment (start 122.0235 112.9265) (end 122.936 112.014) (width 0.3) (layer "F.Cu") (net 14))
 (segment (start 125.476 115) (end 125.603 115.127) (width 0.3) (layer "F.Cu") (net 14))
 (segment (start 125.476 112.395) (end 125.476 115) (width 0.3) (layer "F.Cu") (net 14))
 (segment (start 121.793 112.9265) (end 122.0235 112.9265) (width 0.3) (layer "F.Cu") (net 14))
 (segment (start 124.333 115.127) (end 124.333 112.9265) (width 0.3) (layer "F.Cu") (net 4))
 (segment (start 126.873 113.0535) (end 127 112.9265) (width 0.3) (layer "F.Cu") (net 9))
 (segment (start 126.873 115.127) (end 126.873 113.0535) (width 0.3) (layer "F.Cu") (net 9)))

